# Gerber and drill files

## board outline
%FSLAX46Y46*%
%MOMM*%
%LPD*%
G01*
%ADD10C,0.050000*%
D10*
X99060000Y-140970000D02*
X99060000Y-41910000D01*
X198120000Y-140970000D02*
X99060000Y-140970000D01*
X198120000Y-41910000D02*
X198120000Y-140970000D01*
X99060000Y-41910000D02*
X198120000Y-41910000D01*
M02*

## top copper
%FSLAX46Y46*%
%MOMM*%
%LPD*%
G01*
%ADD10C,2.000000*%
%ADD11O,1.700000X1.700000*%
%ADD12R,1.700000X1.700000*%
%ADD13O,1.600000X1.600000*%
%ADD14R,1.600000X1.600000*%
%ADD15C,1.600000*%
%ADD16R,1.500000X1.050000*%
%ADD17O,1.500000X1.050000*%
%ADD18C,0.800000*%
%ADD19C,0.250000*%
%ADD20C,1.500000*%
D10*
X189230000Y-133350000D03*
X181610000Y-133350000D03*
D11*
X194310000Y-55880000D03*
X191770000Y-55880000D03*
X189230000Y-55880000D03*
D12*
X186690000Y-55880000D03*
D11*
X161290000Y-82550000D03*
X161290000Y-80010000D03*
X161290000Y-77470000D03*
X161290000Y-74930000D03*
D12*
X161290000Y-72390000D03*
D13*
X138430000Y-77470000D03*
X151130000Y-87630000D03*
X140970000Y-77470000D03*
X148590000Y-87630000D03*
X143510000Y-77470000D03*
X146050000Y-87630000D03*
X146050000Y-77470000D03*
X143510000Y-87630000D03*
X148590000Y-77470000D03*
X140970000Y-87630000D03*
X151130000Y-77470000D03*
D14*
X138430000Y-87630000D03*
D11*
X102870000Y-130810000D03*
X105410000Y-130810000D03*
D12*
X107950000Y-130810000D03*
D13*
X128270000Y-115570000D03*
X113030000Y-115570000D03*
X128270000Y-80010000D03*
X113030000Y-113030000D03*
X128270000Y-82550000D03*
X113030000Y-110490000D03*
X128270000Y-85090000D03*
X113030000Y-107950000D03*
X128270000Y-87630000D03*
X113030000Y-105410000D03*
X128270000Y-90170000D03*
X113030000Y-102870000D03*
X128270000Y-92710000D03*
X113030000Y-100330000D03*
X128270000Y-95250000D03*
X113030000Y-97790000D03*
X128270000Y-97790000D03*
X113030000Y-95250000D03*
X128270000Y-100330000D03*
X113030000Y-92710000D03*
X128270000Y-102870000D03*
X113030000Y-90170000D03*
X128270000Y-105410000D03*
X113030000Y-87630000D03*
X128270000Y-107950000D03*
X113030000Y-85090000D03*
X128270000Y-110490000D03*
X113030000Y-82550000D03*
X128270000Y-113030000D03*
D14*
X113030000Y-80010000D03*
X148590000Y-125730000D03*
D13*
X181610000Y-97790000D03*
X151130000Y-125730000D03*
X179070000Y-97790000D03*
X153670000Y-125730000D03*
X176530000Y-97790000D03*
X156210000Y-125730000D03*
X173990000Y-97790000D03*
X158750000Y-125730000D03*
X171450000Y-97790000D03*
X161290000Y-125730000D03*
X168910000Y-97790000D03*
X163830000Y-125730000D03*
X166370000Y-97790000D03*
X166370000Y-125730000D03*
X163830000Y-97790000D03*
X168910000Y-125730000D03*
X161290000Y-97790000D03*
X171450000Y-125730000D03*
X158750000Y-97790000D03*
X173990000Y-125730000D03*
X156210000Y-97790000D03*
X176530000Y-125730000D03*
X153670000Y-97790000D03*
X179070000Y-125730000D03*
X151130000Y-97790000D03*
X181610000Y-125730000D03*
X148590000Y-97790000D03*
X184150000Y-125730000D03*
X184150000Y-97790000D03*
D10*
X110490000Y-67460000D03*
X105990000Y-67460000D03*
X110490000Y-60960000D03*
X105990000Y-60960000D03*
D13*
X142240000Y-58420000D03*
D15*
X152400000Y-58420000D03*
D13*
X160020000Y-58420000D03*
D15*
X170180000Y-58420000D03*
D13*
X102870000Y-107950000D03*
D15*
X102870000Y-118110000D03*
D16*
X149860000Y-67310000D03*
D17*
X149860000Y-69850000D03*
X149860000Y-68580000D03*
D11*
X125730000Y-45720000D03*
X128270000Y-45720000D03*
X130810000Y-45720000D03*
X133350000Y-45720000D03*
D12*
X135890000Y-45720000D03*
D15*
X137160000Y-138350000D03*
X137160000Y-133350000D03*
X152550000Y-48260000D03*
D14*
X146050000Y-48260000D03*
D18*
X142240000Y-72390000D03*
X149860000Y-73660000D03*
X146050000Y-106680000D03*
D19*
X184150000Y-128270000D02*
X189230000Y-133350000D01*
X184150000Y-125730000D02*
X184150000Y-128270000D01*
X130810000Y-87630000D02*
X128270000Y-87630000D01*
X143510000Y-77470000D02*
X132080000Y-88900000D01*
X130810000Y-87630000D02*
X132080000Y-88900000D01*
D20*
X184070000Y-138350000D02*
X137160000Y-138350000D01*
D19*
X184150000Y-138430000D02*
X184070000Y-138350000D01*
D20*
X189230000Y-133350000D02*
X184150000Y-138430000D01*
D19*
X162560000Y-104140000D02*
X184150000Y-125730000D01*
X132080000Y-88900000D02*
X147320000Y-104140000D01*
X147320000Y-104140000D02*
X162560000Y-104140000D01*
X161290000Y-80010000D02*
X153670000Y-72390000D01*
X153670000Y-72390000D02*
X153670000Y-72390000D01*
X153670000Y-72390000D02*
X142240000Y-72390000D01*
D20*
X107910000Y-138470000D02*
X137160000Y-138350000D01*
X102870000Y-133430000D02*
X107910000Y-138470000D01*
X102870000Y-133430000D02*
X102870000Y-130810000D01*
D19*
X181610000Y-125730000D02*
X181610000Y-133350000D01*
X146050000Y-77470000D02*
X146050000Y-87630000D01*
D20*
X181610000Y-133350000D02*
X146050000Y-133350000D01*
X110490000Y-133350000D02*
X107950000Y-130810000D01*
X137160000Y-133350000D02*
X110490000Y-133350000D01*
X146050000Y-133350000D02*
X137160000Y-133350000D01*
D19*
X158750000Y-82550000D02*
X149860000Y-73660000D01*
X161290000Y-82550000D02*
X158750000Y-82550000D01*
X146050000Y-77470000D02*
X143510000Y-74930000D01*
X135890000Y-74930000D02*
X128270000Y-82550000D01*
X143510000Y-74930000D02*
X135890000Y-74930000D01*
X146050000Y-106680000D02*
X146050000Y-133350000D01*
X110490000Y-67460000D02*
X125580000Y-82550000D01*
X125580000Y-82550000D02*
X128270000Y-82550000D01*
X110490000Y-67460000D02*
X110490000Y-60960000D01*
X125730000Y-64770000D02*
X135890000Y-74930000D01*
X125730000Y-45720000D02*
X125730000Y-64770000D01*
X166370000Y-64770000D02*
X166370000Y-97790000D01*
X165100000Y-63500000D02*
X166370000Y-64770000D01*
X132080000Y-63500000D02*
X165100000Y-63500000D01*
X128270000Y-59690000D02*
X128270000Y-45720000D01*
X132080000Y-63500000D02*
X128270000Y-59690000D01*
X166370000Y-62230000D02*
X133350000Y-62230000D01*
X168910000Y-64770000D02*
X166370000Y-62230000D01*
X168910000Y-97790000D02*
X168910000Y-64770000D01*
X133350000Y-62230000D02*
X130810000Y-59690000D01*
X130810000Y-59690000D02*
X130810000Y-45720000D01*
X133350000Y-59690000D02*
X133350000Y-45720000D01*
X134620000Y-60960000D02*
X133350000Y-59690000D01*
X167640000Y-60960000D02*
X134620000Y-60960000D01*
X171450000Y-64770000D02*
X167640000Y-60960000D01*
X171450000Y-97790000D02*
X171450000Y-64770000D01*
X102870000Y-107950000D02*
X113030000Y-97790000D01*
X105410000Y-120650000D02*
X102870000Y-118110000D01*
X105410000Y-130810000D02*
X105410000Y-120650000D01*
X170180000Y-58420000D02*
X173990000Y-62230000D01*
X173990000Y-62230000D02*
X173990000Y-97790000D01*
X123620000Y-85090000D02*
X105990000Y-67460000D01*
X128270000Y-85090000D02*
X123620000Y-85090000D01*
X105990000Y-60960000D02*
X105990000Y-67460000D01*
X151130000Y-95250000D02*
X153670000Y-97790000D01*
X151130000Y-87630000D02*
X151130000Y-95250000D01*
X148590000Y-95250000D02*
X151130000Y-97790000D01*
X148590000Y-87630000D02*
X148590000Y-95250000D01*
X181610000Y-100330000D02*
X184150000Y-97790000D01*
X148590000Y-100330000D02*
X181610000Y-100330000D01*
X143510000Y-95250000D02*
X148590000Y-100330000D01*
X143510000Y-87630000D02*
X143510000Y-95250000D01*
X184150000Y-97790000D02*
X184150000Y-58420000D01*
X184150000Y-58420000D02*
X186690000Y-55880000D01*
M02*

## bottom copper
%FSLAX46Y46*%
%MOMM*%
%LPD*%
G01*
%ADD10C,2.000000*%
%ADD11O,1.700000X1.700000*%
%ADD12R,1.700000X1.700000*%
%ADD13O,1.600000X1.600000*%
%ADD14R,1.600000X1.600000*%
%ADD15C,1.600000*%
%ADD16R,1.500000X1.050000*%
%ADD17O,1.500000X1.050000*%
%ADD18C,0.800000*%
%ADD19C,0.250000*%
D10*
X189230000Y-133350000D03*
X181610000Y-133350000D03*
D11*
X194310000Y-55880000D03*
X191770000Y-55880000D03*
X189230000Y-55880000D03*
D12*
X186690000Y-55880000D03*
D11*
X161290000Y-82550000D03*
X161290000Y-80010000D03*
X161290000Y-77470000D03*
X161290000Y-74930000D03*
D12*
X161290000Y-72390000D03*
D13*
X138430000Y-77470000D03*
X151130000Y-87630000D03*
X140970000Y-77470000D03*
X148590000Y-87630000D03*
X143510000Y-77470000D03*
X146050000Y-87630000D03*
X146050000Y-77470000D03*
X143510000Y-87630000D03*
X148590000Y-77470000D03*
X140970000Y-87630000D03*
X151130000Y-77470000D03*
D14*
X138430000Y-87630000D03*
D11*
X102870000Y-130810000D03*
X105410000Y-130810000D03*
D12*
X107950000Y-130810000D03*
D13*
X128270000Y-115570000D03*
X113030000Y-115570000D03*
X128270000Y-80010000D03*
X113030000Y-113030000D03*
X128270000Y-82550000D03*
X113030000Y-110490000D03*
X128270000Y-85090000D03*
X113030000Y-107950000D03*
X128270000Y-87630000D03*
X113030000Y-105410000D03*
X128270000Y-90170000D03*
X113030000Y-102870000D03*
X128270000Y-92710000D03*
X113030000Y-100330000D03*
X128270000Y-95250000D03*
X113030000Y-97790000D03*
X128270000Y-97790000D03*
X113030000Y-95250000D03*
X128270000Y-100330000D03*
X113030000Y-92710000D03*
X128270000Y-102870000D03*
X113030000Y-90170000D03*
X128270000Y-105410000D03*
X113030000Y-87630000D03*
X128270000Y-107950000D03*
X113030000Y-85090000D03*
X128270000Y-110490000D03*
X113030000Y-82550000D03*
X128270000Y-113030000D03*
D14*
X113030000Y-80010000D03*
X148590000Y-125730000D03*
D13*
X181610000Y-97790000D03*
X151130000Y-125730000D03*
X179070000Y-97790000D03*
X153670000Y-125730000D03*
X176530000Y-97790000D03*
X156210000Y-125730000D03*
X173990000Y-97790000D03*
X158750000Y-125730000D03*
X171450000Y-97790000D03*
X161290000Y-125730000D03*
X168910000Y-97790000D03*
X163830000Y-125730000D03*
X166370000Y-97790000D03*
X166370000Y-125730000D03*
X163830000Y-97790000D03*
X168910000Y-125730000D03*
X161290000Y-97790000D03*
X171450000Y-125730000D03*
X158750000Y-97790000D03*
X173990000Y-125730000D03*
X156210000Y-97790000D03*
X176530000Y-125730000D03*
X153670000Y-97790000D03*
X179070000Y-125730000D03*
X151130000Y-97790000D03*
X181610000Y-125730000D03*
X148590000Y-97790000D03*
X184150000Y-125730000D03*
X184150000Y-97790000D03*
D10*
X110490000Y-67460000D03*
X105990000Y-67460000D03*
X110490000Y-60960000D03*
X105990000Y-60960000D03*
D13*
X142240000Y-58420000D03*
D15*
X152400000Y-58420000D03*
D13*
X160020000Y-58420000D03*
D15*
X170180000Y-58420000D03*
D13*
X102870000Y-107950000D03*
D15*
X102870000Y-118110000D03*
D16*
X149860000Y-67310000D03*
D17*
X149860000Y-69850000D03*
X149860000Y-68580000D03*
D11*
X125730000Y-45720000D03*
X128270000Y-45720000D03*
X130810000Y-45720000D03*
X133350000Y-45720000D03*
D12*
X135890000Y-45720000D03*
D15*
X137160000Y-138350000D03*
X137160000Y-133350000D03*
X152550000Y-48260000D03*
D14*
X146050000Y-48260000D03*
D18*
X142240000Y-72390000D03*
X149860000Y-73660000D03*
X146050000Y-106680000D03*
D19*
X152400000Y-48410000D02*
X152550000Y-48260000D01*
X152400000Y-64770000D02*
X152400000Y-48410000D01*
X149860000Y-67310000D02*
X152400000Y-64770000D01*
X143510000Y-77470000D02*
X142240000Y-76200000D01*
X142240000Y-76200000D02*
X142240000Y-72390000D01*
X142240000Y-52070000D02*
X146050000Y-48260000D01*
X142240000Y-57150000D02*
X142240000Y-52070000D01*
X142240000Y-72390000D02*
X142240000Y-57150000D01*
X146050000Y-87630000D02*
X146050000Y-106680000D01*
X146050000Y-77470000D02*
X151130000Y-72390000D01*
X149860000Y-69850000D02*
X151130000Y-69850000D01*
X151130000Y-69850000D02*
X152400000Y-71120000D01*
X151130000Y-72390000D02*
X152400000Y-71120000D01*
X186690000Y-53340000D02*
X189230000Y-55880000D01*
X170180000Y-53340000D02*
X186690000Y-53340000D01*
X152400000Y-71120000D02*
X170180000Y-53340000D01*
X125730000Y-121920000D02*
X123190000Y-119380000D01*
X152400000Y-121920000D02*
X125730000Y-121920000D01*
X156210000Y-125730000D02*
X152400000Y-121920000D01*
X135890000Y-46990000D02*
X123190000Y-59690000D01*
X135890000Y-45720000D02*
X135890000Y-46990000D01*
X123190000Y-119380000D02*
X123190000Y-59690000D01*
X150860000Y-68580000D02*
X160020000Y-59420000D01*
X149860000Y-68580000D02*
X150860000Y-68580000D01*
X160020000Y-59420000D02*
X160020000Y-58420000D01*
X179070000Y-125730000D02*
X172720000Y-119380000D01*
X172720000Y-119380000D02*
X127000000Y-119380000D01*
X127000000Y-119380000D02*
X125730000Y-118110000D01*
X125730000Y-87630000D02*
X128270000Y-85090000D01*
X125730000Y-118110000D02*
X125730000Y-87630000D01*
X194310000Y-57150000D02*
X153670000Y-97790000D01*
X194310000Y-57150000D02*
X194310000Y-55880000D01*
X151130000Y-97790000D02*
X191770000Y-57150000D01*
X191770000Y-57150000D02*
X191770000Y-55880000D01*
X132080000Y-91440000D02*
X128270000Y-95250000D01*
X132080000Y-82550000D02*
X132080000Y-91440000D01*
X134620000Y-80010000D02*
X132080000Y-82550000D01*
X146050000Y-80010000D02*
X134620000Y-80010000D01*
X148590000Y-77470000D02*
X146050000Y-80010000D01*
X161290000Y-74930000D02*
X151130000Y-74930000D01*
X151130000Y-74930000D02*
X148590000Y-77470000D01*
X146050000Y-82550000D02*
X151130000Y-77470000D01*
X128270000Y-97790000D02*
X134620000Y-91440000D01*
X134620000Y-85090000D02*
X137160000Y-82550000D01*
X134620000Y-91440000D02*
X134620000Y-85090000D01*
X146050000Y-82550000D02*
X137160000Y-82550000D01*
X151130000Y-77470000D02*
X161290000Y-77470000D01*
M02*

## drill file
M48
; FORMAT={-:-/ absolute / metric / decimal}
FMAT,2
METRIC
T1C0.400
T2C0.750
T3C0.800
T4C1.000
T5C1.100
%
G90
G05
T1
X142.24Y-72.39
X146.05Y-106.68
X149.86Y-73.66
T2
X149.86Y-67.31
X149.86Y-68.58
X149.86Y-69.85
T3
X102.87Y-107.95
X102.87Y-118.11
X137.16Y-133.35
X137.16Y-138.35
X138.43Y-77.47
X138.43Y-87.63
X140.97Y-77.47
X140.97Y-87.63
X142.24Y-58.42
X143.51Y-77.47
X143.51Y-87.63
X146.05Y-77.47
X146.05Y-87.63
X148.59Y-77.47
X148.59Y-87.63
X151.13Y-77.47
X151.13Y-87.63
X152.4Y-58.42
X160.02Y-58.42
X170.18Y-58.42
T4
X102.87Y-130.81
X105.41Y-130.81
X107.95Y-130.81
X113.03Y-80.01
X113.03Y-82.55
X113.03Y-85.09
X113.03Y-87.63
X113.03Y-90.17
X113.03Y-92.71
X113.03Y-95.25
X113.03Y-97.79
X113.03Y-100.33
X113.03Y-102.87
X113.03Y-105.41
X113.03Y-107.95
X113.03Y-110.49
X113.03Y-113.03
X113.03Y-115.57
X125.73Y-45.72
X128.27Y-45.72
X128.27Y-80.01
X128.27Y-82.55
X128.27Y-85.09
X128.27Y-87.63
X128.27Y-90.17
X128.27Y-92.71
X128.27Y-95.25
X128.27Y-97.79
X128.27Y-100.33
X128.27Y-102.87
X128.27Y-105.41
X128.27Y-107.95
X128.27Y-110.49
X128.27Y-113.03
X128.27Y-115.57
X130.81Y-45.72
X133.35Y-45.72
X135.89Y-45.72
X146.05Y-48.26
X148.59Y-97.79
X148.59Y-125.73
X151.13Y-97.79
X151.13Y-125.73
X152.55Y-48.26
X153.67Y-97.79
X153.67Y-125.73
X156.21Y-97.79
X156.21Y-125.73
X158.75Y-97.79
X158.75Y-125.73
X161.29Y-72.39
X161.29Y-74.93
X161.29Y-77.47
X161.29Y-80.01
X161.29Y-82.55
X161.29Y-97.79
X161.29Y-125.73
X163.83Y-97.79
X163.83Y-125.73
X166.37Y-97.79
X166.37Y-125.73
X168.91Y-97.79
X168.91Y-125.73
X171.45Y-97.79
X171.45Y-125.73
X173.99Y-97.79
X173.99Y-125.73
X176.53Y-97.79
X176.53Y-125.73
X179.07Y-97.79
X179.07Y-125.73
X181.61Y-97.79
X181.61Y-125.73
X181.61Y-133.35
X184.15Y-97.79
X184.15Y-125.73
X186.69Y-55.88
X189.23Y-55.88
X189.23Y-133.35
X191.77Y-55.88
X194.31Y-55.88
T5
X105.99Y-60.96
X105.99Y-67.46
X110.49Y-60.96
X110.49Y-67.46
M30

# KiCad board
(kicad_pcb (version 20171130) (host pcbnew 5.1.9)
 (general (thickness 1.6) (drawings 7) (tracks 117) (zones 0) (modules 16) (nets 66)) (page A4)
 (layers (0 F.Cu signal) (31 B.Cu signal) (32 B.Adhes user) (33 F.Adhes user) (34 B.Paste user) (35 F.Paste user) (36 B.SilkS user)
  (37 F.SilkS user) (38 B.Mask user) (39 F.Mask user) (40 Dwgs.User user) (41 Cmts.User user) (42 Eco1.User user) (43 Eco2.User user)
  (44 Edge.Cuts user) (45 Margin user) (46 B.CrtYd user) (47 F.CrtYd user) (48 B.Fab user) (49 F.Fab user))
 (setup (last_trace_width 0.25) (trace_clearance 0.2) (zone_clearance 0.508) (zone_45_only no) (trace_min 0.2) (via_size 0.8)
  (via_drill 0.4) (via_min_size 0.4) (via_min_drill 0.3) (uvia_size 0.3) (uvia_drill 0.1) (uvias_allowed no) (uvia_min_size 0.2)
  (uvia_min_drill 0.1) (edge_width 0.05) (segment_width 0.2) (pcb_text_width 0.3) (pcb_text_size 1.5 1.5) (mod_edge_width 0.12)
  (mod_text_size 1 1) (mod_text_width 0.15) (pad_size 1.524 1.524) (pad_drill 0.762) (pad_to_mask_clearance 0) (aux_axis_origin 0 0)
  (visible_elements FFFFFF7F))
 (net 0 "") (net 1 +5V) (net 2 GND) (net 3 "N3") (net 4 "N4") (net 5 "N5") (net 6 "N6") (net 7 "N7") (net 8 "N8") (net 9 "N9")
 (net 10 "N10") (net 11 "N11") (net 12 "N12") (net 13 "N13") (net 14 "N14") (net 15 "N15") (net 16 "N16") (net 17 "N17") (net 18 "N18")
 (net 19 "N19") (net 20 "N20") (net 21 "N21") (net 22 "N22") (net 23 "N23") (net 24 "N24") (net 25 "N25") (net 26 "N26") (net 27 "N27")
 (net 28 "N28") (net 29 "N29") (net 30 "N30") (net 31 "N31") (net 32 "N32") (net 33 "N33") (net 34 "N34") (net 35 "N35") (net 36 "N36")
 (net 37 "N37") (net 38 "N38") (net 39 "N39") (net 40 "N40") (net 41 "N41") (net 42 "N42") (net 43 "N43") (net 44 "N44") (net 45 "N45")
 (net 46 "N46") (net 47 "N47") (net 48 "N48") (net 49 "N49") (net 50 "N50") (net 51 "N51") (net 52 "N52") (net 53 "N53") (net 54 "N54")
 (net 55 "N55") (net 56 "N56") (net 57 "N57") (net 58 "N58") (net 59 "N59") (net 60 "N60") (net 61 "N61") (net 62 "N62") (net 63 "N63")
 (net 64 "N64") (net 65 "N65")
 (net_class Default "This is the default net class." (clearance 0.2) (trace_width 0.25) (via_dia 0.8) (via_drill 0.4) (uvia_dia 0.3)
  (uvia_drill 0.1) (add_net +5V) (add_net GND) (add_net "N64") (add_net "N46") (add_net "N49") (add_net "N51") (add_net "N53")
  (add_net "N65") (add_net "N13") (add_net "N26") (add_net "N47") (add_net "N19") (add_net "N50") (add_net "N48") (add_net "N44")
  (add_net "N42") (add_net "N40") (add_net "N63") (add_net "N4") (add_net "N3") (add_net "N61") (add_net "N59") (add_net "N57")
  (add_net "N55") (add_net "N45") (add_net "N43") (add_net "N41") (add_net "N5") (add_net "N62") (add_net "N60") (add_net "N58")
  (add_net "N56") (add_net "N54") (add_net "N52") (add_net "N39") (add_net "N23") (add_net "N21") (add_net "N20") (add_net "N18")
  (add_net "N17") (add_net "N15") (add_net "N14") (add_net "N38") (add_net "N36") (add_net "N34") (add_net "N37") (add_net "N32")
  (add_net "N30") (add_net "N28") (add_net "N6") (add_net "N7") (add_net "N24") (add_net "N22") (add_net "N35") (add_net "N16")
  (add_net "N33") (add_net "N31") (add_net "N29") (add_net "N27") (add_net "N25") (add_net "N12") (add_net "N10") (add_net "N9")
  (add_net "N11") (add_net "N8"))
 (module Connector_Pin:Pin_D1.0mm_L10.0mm (layer F.Cu) (at 189.23 133.35)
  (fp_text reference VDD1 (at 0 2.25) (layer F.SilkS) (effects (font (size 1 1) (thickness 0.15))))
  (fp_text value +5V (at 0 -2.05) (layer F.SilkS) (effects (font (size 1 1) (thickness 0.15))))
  (pad 1 thru_hole circle (at 0 0) (size 2 2) (drill 1) (layers *.Cu *.Mask) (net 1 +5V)))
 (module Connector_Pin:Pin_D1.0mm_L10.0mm (layer F.Cu) (at 181.61 133.35)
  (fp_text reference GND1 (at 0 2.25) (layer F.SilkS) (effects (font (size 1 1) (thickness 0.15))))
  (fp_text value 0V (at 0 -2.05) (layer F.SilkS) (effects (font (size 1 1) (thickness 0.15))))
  (pad 1 thru_hole circle (at 0 0) (size 2 2) (drill 1) (layers *.Cu *.Mask) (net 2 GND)))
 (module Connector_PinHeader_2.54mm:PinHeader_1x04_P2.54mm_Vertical (layer F.Cu) (at 186.69 55.88 90)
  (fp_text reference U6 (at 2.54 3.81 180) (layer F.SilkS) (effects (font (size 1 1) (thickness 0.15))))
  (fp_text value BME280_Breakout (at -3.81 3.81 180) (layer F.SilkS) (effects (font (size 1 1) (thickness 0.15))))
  (pad 4 thru_hole oval (at 0 7.62 90) (size 1.7 1.7) (drill 1) (layers *.Cu *.Mask) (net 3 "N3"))
  (pad 3 thru_hole oval (at 0 5.08 90) (size 1.7 1.7) (drill 1) (layers *.Cu *.Mask) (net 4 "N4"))
  (pad 2 thru_hole oval (at 0 2.54 90) (size 1.7 1.7) (drill 1) (layers *.Cu *.Mask) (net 2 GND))
  (pad 1 thru_hole rect (at 0 0 90) (size 1.7 1.7) (drill 1) (layers *.Cu *.Mask) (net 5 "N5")))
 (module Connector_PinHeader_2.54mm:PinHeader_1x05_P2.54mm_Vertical (layer F.Cu) (at 161.29 72.39)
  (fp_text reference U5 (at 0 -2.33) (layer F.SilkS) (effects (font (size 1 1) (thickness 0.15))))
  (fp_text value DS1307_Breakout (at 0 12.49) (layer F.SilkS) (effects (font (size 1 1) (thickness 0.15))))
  (pad 5 thru_hole oval (at 0 10.16) (size 1.7 1.7) (drill 1) (layers *.Cu *.Mask) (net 2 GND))
  (pad 4 thru_hole oval (at 0 7.62) (size 1.7 1.7) (drill 1) (layers *.Cu *.Mask) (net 1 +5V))
  (pad 3 thru_hole oval (at 0 5.08) (size 1.7 1.7) (drill 1) (layers *.Cu *.Mask) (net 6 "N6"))
  (pad 2 thru_hole oval (at 0 2.54) (size 1.7 1.7) (drill 1) (layers *.Cu *.Mask) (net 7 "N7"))
  (pad 1 thru_hole rect (at 0 0) (size 1.7 1.7) (drill 1) (layers *.Cu *.Mask) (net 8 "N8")))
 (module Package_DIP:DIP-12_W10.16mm (layer F.Cu) (at 138.43 87.63 90)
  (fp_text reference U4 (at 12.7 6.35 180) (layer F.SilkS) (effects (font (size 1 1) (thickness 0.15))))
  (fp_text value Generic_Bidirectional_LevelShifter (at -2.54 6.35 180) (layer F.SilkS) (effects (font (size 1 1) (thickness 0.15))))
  (pad 12 thru_hole oval (at 10.16 0 90) (size 1.6 1.6) (drill 0.8) (layers *.Cu *.Mask) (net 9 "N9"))
  (pad 6 thru_hole oval (at 0 12.7 90) (size 1.6 1.6) (drill 0.8) (layers *.Cu *.Mask) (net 3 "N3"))
  (pad 11 thru_hole oval (at 10.16 2.54 90) (size 1.6 1.6) (drill 0.8) (layers *.Cu *.Mask) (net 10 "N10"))
  (pad 5 thru_hole oval (at 0 10.16 90) (size 1.6 1.6) (drill 0.8) (layers *.Cu *.Mask) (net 4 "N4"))
  (pad 10 thru_hole oval (at 10.16 5.08 90) (size 1.6 1.6) (drill 0.8) (layers *.Cu *.Mask) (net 1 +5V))
  (pad 4 thru_hole oval (at 0 7.62 90) (size 1.6 1.6) (drill 0.8) (layers *.Cu *.Mask) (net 2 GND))
  (pad 9 thru_hole oval (at 10.16 7.62 90) (size 1.6 1.6) (drill 0.8) (layers *.Cu *.Mask) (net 2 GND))
  (pad 3 thru_hole oval (at 0 5.08 90) (size 1.6 1.6) (drill 0.8) (layers *.Cu *.Mask) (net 5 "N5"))
  (pad 8 thru_hole oval (at 10.16 10.16 90) (size 1.6 1.6) (drill 0.8) (layers *.Cu *.Mask) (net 7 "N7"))
  (pad 2 thru_hole oval (at 0 2.54 90) (size 1.6 1.6) (drill 0.8) (layers *.Cu *.Mask) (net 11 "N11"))
  (pad 7 thru_hole oval (at 10.16 12.7 90) (size 1.6 1.6) (drill 0.8) (layers *.Cu *.Mask) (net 6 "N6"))
  (pad 1 thru_hole rect (at 0 0 90) (size 1.6 1.6) (drill 0.8) (layers *.Cu *.Mask) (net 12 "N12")))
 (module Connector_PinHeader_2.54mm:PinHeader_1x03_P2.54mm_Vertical (layer F.Cu) (at 107.95 130.81 270)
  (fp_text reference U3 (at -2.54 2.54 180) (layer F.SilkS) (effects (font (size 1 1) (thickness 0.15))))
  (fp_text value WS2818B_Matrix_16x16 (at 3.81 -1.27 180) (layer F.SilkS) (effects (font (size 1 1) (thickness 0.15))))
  (pad 3 thru_hole oval (at 0 5.08 270) (size 1.7 1.7) (drill 1) (layers *.Cu *.Mask) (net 1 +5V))
  (pad 2 thru_hole oval (at 0 2.54 270) (size 1.7 1.7) (drill 1) (layers *.Cu *.Mask) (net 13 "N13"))
  (pad 1 thru_hole rect (at 0 0 270) (size 1.7 1.7) (drill 1) (layers *.Cu *.Mask) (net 2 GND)))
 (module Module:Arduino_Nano (layer F.Cu) (at 113.03 80.01)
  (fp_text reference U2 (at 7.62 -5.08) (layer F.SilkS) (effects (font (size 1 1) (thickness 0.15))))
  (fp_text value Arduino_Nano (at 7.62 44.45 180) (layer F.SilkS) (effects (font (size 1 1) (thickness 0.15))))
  (pad 16 thru_hole oval (at 15.24 35.56) (size 1.6 1.6) (drill 1) (layers *.Cu *.Mask) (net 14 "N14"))
  (pad 15 thru_hole oval (at 0 35.56) (size 1.6 1.6) (drill 1) (layers *.Cu *.Mask) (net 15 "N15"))
  (pad 30 thru_hole oval (at 15.24 0) (size 1.6 1.6) (drill 1) (layers *.Cu *.Mask) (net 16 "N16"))
  (pad 14 thru_hole oval (at 0 33.02) (size 1.6 1.6) (drill 1) (layers *.Cu *.Mask) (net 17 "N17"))
  (pad 29 thru_hole oval (at 15.24 2.54) (size 1.6 1.6) (drill 1) (layers *.Cu *.Mask) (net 2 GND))
  (pad 13 thru_hole oval (at 0 30.48) (size 1.6 1.6) (drill 1) (layers *.Cu *.Mask) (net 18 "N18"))
  (pad 28 thru_hole oval (at 15.24 5.08) (size 1.6 1.6) (drill 1) (layers *.Cu *.Mask) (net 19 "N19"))
  (pad 12 thru_hole oval (at 0 27.94) (size 1.6 1.6) (drill 1) (layers *.Cu *.Mask) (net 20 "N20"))
  (pad 27 thru_hole oval (at 15.24 7.62) (size 1.6 1.6) (drill 1) (layers *.Cu *.Mask) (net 1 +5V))
  (pad 11 thru_hole oval (at 0 25.4) (size 1.6 1.6) (drill 1) (layers *.Cu *.Mask) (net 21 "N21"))
  (pad 26 thru_hole oval (at 15.24 10.16) (size 1.6 1.6) (drill 1) (layers *.Cu *.Mask) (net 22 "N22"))
  (pad 10 thru_hole oval (at 0 22.86) (size 1.6 1.6) (drill 1) (layers *.Cu *.Mask) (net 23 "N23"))
  (pad 25 thru_hole oval (at 15.24 12.7) (size 1.6 1.6) (drill 1) (layers *.Cu *.Mask) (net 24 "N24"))
  (pad 9 thru_hole oval (at 0 20.32) (size 1.6 1.6) (drill 1) (layers *.Cu *.Mask) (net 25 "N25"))
  (pad 24 thru_hole oval (at 15.24 15.24) (size 1.6 1.6) (drill 1) (layers *.Cu *.Mask) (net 7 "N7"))
  (pad 8 thru_hole oval (at 0 17.78) (size 1.6 1.6) (drill 1) (layers *.Cu *.Mask) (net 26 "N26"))
  (pad 23 thru_hole oval (at 15.24 17.78) (size 1.6 1.6) (drill 1) (layers *.Cu *.Mask) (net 6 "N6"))
  (pad 7 thru_hole oval (at 0 15.24) (size 1.6 1.6) (drill 1) (layers *.Cu *.Mask) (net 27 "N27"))
  (pad 22 thru_hole oval (at 15.24 20.32) (size 1.6 1.6) (drill 1) (layers *.Cu *.Mask) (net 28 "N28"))
  (pad 6 thru_hole oval (at 0 12.7) (size 1.6 1.6) (drill 1) (layers *.Cu *.Mask) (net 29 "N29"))
  (pad 21 thru_hole oval (at 15.24 22.86) (size 1.6 1.6) (drill 1) (layers *.Cu *.Mask) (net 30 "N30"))
  (pad 5 thru_hole oval (at 0 10.16) (size 1.6 1.6) (drill 1) (layers *.Cu *.Mask) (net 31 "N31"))
  (pad 20 thru_hole oval (at 15.24 25.4) (size 1.6 1.6) (drill 1) (layers *.Cu *.Mask) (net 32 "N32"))
  (pad 4 thru_hole oval (at 0 7.62) (size 1.6 1.6) (drill 1) (layers *.Cu *.Mask) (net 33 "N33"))
  (pad 19 thru_hole oval (at 15.24 27.94) (size 1.6 1.6) (drill 1) (layers *.Cu *.Mask) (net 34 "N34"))
  (pad 3 thru_hole oval (at 0 5.08) (size 1.6 1.6) (drill 1) (layers *.Cu *.Mask) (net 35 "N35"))
  (pad 18 thru_hole oval (at 15.24 30.48) (size 1.6 1.6) (drill 1) (layers *.Cu *.Mask) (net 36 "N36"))
  (pad 2 thru_hole oval (at 0 2.54) (size 1.6 1.6) (drill 1) (layers *.Cu *.Mask) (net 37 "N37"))
  (pad 17 thru_hole oval (at 15.24 33.02) (size 1.6 1.6) (drill 1) (layers *.Cu *.Mask) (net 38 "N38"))
  (pad 1 thru_hole rect (at 0 0) (size 1.6 1.6) (drill 1) (layers *.Cu *.Mask) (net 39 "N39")))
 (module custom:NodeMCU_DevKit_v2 (layer F.Cu) (at 148.59 125.73 90)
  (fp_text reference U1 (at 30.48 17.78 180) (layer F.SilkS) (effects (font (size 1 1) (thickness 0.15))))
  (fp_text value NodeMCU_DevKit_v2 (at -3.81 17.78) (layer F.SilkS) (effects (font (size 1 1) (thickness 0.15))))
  (pad 15 thru_hole rect (at 0 0 90) (size 1.6 1.6) (drill 1) (layers *.Cu *.Mask) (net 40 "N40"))
  (pad 29 thru_hole oval (at 27.94 33.02 90) (size 1.6 1.6) (drill 1) (layers *.Cu *.Mask) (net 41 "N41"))
  (pad 14 thru_hole oval (at 0 2.54 90) (size 1.6 1.6) (drill 1) (layers *.Cu *.Mask) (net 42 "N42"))
  (pad 28 thru_hole oval (at 27.94 30.48 90) (size 1.6 1.6) (drill 1) (layers *.Cu *.Mask) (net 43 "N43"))
  (pad 13 thru_hole oval (at 0 5.08 90) (size 1.6 1.6) (drill 1) (layers *.Cu *.Mask) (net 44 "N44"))
  (pad 27 thru_hole oval (at 27.94 27.94 90) (size 1.6 1.6) (drill 1) (layers *.Cu *.Mask) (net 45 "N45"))
  (pad 12 thru_hole oval (at 0 7.62 90) (size 1.6 1.6) (drill 1) (layers *.Cu *.Mask) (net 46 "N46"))
  (pad 26 thru_hole oval (at 27.94 25.4 90) (size 1.6 1.6) (drill 1) (layers *.Cu *.Mask) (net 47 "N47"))
  (pad 11 thru_hole oval (at 0 10.16 90) (size 1.6 1.6) (drill 1) (layers *.Cu *.Mask) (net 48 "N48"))
  (pad 25 thru_hole oval (at 27.94 22.86 90) (size 1.6 1.6) (drill 1) (layers *.Cu *.Mask) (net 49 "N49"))
  (pad 10 thru_hole oval (at 0 12.7 90) (size 1.6 1.6) (drill 1) (layers *.Cu *.Mask) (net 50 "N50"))
  (pad 24 thru_hole oval (at 27.94 20.32 90) (size 1.6 1.6) (drill 1) (layers *.Cu *.Mask) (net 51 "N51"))
  (pad 9 thru_hole oval (at 0 15.24 90) (size 1.6 1.6) (drill 1) (layers *.Cu *.Mask) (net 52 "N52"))
  (pad 23 thru_hole oval (at 27.94 17.78 90) (size 1.6 1.6) (drill 1) (layers *.Cu *.Mask) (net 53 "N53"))
  (pad 8 thru_hole oval (at 0 17.78 90) (size 1.6 1.6) (drill 1) (layers *.Cu *.Mask) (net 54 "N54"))
  (pad 22 thru_hole oval (at 27.94 15.24 90) (size 1.6 1.6) (drill 1) (layers *.Cu *.Mask) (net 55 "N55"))
  (pad 7 thru_hole oval (at 0 20.32 90) (size 1.6 1.6) (drill 1) (layers *.Cu *.Mask) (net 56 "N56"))
  (pad 21 thru_hole oval (at 27.94 12.7 90) (size 1.6 1.6) (drill 1) (layers *.Cu *.Mask) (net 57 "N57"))
  (pad 6 thru_hole oval (at 0 22.86 90) (size 1.6 1.6) (drill 1) (layers *.Cu *.Mask) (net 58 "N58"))
  (pad 20 thru_hole oval (at 27.94 10.16 90) (size 1.6 1.6) (drill 1) (layers *.Cu *.Mask) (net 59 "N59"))
  (pad 5 thru_hole oval (at 0 25.4 90) (size 1.6 1.6) (drill 1) (layers *.Cu *.Mask) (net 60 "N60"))
  (pad 19 thru_hole oval (at 27.94 7.62 90) (size 1.6 1.6) (drill 1) (layers *.Cu *.Mask) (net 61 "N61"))
  (pad 4 thru_hole oval (at 0 27.94 90) (size 1.6 1.6) (drill 1) (layers *.Cu *.Mask) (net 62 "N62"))
  (pad 18 thru_hole oval (at 27.94 5.08 90) (size 1.6 1.6) (drill 1) (layers *.Cu *.Mask) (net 3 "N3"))
  (pad 3 thru_hole oval (at 0 30.48 90) (size 1.6 1.6) (drill 1) (layers *.Cu *.Mask) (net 19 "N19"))
  (pad 17 thru_hole oval (at 27.94 2.54 90) (size 1.6 1.6) (drill 1) (layers *.Cu *.Mask) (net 4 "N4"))
  (pad 2 thru_hole oval (at 0 33.02 90) (size 1.6 1.6) (drill 1) (layers *.Cu *.Mask) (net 2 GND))
  (pad 16 thru_hole oval (at 27.94 0 90) (size 1.6 1.6) (drill 1) (layers *.Cu *.Mask) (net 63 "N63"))
  (pad 1 thru_hole oval (at 0 35.56 90) (size 1.6 1.6) (drill 1) (layers *.Cu *.Mask) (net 1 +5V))
  (pad 30 thru_hole oval (at 27.94 35.56 90) (size 1.6 1.6) (drill 1) (layers *.Cu *.Mask) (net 5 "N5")))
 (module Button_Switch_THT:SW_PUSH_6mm (layer F.Cu) (at 110.49 60.96 270)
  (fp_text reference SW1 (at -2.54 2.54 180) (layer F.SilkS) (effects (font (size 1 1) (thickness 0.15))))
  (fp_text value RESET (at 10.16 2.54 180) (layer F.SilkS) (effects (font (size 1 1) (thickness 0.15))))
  (pad 1 thru_hole circle (at 6.5 0) (size 2 2) (drill 1.1) (layers *.Cu *.Mask) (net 2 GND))
  (pad 2 thru_hole circle (at 6.5 4.5) (size 2 2) (drill 1.1) (layers *.Cu *.Mask) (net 19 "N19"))
  (pad 1 thru_hole circle (at 0 0) (size 2 2) (drill 1.1) (layers *.Cu *.Mask) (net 2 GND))
  (pad 2 thru_hole circle (at 0 4.5) (size 2 2) (drill 1.1) (layers *.Cu *.Mask) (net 19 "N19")))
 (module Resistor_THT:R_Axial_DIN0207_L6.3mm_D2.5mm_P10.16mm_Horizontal (layer F.Cu) (at 152.4 58.42 180)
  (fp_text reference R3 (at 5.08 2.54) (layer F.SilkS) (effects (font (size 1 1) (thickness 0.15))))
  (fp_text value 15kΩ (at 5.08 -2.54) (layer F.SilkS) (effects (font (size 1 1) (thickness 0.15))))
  (pad 2 thru_hole oval (at 10.16 0 180) (size 1.6 1.6) (drill 0.8) (layers *.Cu *.Mask) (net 1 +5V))
  (pad 1 thru_hole circle (at 0 0 180) (size 1.6 1.6) (drill 0.8) (layers *.Cu *.Mask) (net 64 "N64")))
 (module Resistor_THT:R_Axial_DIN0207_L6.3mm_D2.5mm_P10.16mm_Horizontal (layer F.Cu) (at 170.18 58.42 180)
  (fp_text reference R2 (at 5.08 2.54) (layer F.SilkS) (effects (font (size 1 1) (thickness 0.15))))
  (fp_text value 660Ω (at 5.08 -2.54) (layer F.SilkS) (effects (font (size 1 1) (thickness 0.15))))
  (pad 2 thru_hole oval (at 10.16 0 180) (size 1.6 1.6) (drill 0.8) (layers *.Cu *.Mask) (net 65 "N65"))
  (pad 1 thru_hole circle (at 0 0 180) (size 1.6 1.6) (drill 0.8) (layers *.Cu *.Mask) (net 47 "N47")))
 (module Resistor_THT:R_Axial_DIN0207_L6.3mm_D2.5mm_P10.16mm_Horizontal (layer F.Cu) (at 102.87 118.11 90)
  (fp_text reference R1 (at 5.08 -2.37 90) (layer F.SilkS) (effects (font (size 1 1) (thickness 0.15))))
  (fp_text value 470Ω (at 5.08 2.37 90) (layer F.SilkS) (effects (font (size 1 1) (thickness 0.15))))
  (pad 2 thru_hole oval (at 10.16 0 90) (size 1.6 1.6) (drill 0.8) (layers *.Cu *.Mask) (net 26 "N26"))
  (pad 1 thru_hole circle (at 0 0 90) (size 1.6 1.6) (drill 0.8) (layers *.Cu *.Mask) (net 13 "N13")))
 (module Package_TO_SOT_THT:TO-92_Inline (layer F.Cu) (at 149.86 67.31 270)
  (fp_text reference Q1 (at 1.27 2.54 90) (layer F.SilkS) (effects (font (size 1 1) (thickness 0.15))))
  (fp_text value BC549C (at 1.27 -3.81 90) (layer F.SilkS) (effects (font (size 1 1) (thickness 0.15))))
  (pad 1 thru_hole rect (at 0 0 270) (size 1.05 1.5) (drill 0.75) (layers *.Cu *.Mask) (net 64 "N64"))
  (pad 3 thru_hole oval (at 2.54 0 270) (size 1.05 1.5) (drill 0.75) (layers *.Cu *.Mask) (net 2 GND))
  (pad 2 thru_hole oval (at 1.27 0 270) (size 1.05 1.5) (drill 0.75) (layers *.Cu *.Mask) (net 65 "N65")))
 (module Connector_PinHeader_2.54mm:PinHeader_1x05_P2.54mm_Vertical (layer F.Cu) (at 135.89 45.72 270)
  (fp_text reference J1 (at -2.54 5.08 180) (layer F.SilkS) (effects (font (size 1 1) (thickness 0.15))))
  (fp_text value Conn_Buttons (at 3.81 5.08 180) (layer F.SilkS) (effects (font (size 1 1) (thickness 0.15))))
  (pad 5 thru_hole oval (at 0 10.16 270) (size 1.7 1.7) (drill 1) (layers *.Cu *.Mask) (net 2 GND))
  (pad 4 thru_hole oval (at 0 7.62 270) (size 1.7 1.7) (drill 1) (layers *.Cu *.Mask) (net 53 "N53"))
  (pad 3 thru_hole oval (at 0 5.08 270) (size 1.7 1.7) (drill 1) (layers *.Cu *.Mask) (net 51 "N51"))
  (pad 2 thru_hole oval (at 0 2.54 270) (size 1.7 1.7) (drill 1) (layers *.Cu *.Mask) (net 49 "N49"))
  (pad 1 thru_hole rect (at 0 0 270) (size 1.7 1.7) (drill 1) (layers *.Cu *.Mask) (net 46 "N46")))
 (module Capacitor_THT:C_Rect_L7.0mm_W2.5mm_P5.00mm (layer F.Cu) (at 137.16 133.35 270)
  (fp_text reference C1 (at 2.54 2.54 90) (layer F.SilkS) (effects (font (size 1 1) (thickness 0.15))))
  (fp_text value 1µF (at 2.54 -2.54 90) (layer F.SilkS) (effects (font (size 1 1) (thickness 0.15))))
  (pad 2 thru_hole circle (at 5 0 270) (size 1.6 1.6) (drill 0.8) (layers *.Cu *.Mask) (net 1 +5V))
  (pad 1 thru_hole circle (at 0 0 270) (size 1.6 1.6) (drill 0.8) (layers *.Cu *.Mask) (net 2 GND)))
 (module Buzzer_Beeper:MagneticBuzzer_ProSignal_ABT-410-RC (layer F.Cu) (at 146.05 48.26)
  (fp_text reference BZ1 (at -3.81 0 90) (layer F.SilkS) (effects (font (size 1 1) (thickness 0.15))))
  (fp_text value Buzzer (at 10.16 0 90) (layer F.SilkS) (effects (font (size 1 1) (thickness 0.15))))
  (pad 2 thru_hole circle (at 6.5 0) (size 1.6 1.6) (drill 1) (layers *.Cu *.Mask) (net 64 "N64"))
  (pad 1 thru_hole rect (at 0 0) (size 1.6 1.6) (drill 1) (layers *.Cu *.Mask) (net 1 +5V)))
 (gr_line (start 99.06 140.97) (end 99.06 41.91) (layer Edge.Cuts) (width 0.05))
 (gr_line (start 198.12 140.97) (end 99.06 140.97) (layer Edge.Cuts) (width 0.05))
 (gr_line (start 198.12 41.91) (end 198.12 140.97) (layer Edge.Cuts) (width 0.05))
 (gr_line (start 99.06 41.91) (end 198.12 41.91) (layer Edge.Cuts) (width 0.05))
 (segment (start 152.4 48.41) (end 152.55 48.26) (width 0.25) (layer B.Cu) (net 64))
 (segment (start 152.4 64.77) (end 152.4 48.41) (width 0.25) (layer B.Cu) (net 64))
 (segment (start 149.86 67.31) (end 152.4 64.77) (width 0.25) (layer B.Cu) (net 64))
 (segment (start 184.15 128.27) (end 189.23 133.35) (width 0.25) (layer F.Cu) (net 1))
 (segment (start 184.15 125.73) (end 184.15 128.27) (width 0.25) (layer F.Cu) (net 1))
 (segment (start 130.81 87.63) (end 128.27 87.63) (width 0.25) (layer F.Cu) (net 1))
 (segment (start 143.51 77.47) (end 132.08 88.9) (width 0.25) (layer F.Cu) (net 1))
 (segment (start 130.81 87.63) (end 132.08 88.9) (width 0.25) (layer F.Cu) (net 1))
 (segment (start 184.07 138.35) (end 137.16 138.35) (width 1.5) (layer F.Cu) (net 1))
 (segment (start 184.15 138.43) (end 184.07 138.35) (width 0.25) (layer F.Cu) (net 1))
 (segment (start 189.23 133.35) (end 184.15 138.43) (width 1.5) (layer F.Cu) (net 1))
 (segment (start 162.56 104.14) (end 184.15 125.73) (width 0.25) (layer F.Cu) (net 1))
 (segment (start 132.08 88.9) (end 147.32 104.14) (width 0.25) (layer F.Cu) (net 1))
 (segment (start 147.32 104.14) (end 162.56 104.14) (width 0.25) (layer F.Cu) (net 1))
 (segment (start 143.51 77.47) (end 142.24 76.2) (width 0.25) (layer B.Cu) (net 1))
 (segment (start 142.24 76.2) (end 142.24 72.39) (width 0.25) (layer B.Cu) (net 1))
 (segment (start 142.24 52.07) (end 146.05 48.26) (width 0.25) (layer B.Cu) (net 1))
 (segment (start 161.29 80.01) (end 153.67 72.39) (width 0.25) (layer F.Cu) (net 1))
 (segment (start 153.67 72.39) (end 153.67 72.39) (width 0.25) (layer F.Cu) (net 1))
 (via (at 142.24 72.39) (size 0.8) (drill 0.4) (layers F.Cu B.Cu) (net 1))
 (segment (start 153.67 72.39) (end 142.24 72.39) (width 0.25) (layer F.Cu) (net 1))
 (segment (start 107.91 138.47) (end 137.16 138.35) (width 1.5) (layer F.Cu) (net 1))
 (segment (start 102.87 133.43) (end 107.91 138.47) (width 1.5) (layer F.Cu) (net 1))
 (segment (start 102.87 133.43) (end 102.87 130.81) (width 1.5) (layer F.Cu) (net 1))
 (segment (start 142.24 57.15) (end 142.24 52.07) (width 0.25) (layer B.Cu) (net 1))
 (segment (start 142.24 72.39) (end 142.24 57.15) (width 0.25) (layer B.Cu) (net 1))
 (segment (start 181.61 125.73) (end 181.61 133.35) (width 0.25) (layer F.Cu) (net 2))
 (segment (start 146.05 77.47) (end 146.05 87.63) (width 0.25) (layer F.Cu) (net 2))
 (segment (start 181.61 133.35) (end 146.05 133.35) (width 1.5) (layer F.Cu) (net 2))
 (segment (start 110.49 133.35) (end 107.95 130.81) (width 1.5) (layer F.Cu) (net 2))
 (segment (start 137.16 133.35) (end 110.49 133.35) (width 1.5) (layer F.Cu) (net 2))
 (segment (start 146.05 133.35) (end 137.16 133.35) (width 1.5) (layer F.Cu) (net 2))
 (segment (start 146.05 87.63) (end 146.05 106.68) (width 0.25) (layer B.Cu) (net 2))
 (segment (start 146.05 77.47) (end 151.13 72.39) (width 0.25) (layer B.Cu) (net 2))
 (segment (start 149.86 69.85) (end 151.13 69.85) (width 0.25) (layer B.Cu) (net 2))
 (segment (start 151.13 69.85) (end 152.4 71.12) (width 0.25) (layer B.Cu) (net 2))
 (segment (start 151.13 72.39) (end 152.4 71.12) (width 0.25) (layer B.Cu) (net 2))
 (via (at 149.86 73.66) (size 0.8) (drill 0.4) (layers F.Cu B.Cu) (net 2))
 (segment (start 158.75 82.55) (end 149.86 73.66) (width 0.25) (layer F.Cu) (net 2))
 (segment (start 161.29 82.55) (end 158.75 82.55) (width 0.25) (layer F.Cu) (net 2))
 (segment (start 146.05 77.47) (end 143.51 74.93) (width 0.25) (layer F.Cu) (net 2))
 (segment (start 135.89 74.93) (end 128.27 82.55) (width 0.25) (layer F.Cu) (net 2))
 (segment (start 143.51 74.93) (end 135.89 74.93) (width 0.25) (layer F.Cu) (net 2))
 (via (at 146.05 106.68) (size 0.8) (drill 0.4) (layers F.Cu B.Cu) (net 2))
 (segment (start 146.05 106.68) (end 146.05 133.35) (width 0.25) (layer F.Cu) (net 2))
 (segment (start 110.49 67.46) (end 125.58 82.55) (width 0.25) (layer F.Cu) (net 2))
 (segment (start 125.58 82.55) (end 128.27 82.55) (width 0.25) (layer F.Cu) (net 2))
 (segment (start 110.49 67.46) (end 110.49 60.96) (width 0.25) (layer F.Cu) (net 2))
 (segment (start 186.69 53.34) (end 189.23 55.88) (width 0.25) (layer B.Cu) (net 2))
 (segment (start 170.18 53.34) (end 186.69 53.34) (width 0.25) (layer B.Cu) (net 2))
 (segment (start 152.4 71.12) (end 170.18 53.34) (width 0.25) (layer B.Cu) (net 2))
 (segment (start 125.73 64.77) (end 135.89 74.93) (width 0.25) (layer F.Cu) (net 2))
 (segment (start 125.73 45.72) (end 125.73 64.77) (width 0.25) (layer F.Cu) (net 2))
 (segment (start 166.37 64.77) (end 166.37 97.79) (width 0.25) (layer F.Cu) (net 53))
 (segment (start 165.1 63.5) (end 166.37 64.77) (width 0.25) (layer F.Cu) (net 53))
 (segment (start 132.08 63.5) (end 165.1 63.5) (width 0.25) (layer F.Cu) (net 53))
 (segment (start 128.27 59.69) (end 128.27 45.72) (width 0.25) (layer F.Cu) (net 53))
 (segment (start 132.08 63.5) (end 128.27 59.69) (width 0.25) (layer F.Cu) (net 53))
 (segment (start 166.37 62.23) (end 133.35 62.23) (width 0.25) (layer F.Cu) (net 51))
 (segment (start 168.91 64.77) (end 166.37 62.23) (width 0.25) (layer F.Cu) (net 51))
 (segment (start 168.91 97.79) (end 168.91 64.77) (width 0.25) (layer F.Cu) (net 51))
 (segment (start 133.35 62.23) (end 130.81 59.69) (width 0.25) (layer F.Cu) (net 51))
 (segment (start 130.81 59.69) (end 130.81 45.72) (width 0.25) (layer F.Cu) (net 51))
 (segment (start 133.35 59.69) (end 133.35 45.72) (width 0.25) (layer F.Cu) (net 49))
 (segment (start 134.62 60.96) (end 133.35 59.69) (width 0.25) (layer F.Cu) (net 49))
 (segment (start 167.64 60.96) (end 134.62 60.96) (width 0.25) (layer F.Cu) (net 49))
 (segment (start 171.45 64.77) (end 167.64 60.96) (width 0.25) (layer F.Cu) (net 49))
 (segment (start 171.45 97.79) (end 171.45 64.77) (width 0.25) (layer F.Cu) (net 49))
 (segment (start 125.73 121.92) (end 123.19 119.38) (width 0.25) (layer B.Cu) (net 46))
 (segment (start 152.4 121.92) (end 125.73 121.92) (width 0.25) (layer B.Cu) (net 46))
 (segment (start 156.21 125.73) (end 152.4 121.92) (width 0.25) (layer B.Cu) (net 46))
 (segment (start 135.89 46.99) (end 123.19 59.69) (width 0.25) (layer B.Cu) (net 46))
 (segment (start 135.89 45.72) (end 135.89 46.99) (width 0.25) (layer B.Cu) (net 46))
 (segment (start 123.19 119.38) (end 123.19 59.69) (width 0.25) (layer B.Cu) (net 46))
 (segment (start 150.86 68.58) (end 160.02 59.42) (width 0.25) (layer B.Cu) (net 65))
 (segment (start 149.86 68.58) (end 150.86 68.58) (width 0.25) (layer B.Cu) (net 65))
 (segment (start 160.02 59.42) (end 160.02 58.42) (width 0.25) (layer B.Cu) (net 65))
 (segment (start 102.87 107.95) (end 113.03 97.79) (width 0.25) (layer F.Cu) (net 26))
 (segment (start 105.41 120.65) (end 102.87 118.11) (width 0.25) (layer F.Cu) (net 13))
 (segment (start 105.41 130.81) (end 105.41 120.65) (width 0.25) (layer F.Cu) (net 13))
 (segment (start 170.18 58.42) (end 173.99 62.23) (width 0.25) (layer F.Cu) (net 47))
 (segment (start 173.99 62.23) (end 173.99 97.79) (width 0.25) (layer F.Cu) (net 47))
 (segment (start 179.07 125.73) (end 172.72 119.38) (width 0.25) (layer B.Cu) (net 19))
 (segment (start 172.72 119.38) (end 127 119.38) (width 0.25) (layer B.Cu) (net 19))
 (segment (start 127 119.38) (end 125.73 118.11) (width 0.25) (layer B.Cu) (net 19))
 (segment (start 125.73 87.63) (end 128.27 85.09) (width 0.25) (layer B.Cu) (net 19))
 (segment (start 125.73 118.11) (end 125.73 87.63) (width 0.25) (layer B.Cu) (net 19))
 (segment (start 123.62 85.09) (end 105.99 67.46) (width 0.25) (layer F.Cu) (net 19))
 (segment (start 128.27 85.09) (end 123.62 85.09) (width 0.25) (layer F.Cu) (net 19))
 (segment (start 105.99 60.96) (end 105.99 67.46) (width 0.25) (layer F.Cu) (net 19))
 (segment (start 151.13 95.25) (end 153.67 97.79) (width 0.25) (layer F.Cu) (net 3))
 (segment (start 151.13 87.63) (end 151.13 95.25) (width 0.25) (layer F.Cu) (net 3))
 (segment (start 194.31 57.15) (end 153.67 97.79) (width 0.25) (layer B.Cu) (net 3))
 (segment (start 194.31 57.15) (end 194.31 55.88) (width 0.25) (layer B.Cu) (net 3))
 (segment (start 148.59 95.25) (end 151.13 97.79) (width 0.25) (layer F.Cu) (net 4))
 (segment (start 148.59 87.63) (end 148.59 95.25) (width 0.25) (layer F.Cu) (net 4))
 (segment (start 151.13 97.79) (end 191.77 57.15) (width 0.25) (layer B.Cu) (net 4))
 (segment (start 191.77 57.15) (end 191.77 55.88) (width 0.25) (layer B.Cu) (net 4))
 (segment (start 181.61 100.33) (end 184.15 97.79) (width 0.25) (layer F.Cu) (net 5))
 (segment (start 148.59 100.33) (end 181.61 100.33) (width 0.25) (layer F.Cu) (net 5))
 (segment (start 143.51 95.25) (end 148.59 100.33) (width 0.25) (layer F.Cu) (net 5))
 (segment (start 143.51 87.63) (end 143.51 95.25) (width 0.25) (layer F.Cu) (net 5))
 (segment (start 184.15 97.79) (end 184.15 58.42) (width 0.25) (layer F.Cu) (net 5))
 (segment (start 184.15 58.42) (end 186.69 55.88) (width 0.25) (layer F.Cu) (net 5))
 (segment (start 132.08 91.44) (end 128.27 95.25) (width 0.25) (layer B.Cu) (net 7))
 (segment (start 132.08 82.55) (end 132.08 91.44) (width 0.25) (layer B.Cu) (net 7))
 (segment (start 134.62 80.01) (end 132.08 82.55) (width 0.25) (layer B.Cu) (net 7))
 (segment (start 146.05 80.01) (end 134.62 80.01) (width 0.25) (layer B.Cu) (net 7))
 (segment (start 148.59 77.47) (end 146.05 80.01) (width 0.25) (layer B.Cu) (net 7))
 (segment (start 161.29 74.93) (end 151.13 74.93) (width 0.25) (layer B.Cu) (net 7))
 (segment (start 151.13 74.93) (end 148.59 77.47) (width 0.25) (layer B.Cu) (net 7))
 (segment (start 146.05 82.55) (end 151.13 77.47) (width 0.25) (layer B.Cu) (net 6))
 (segment (start 128.27 97.79) (end 134.62 91.44) (width 0.25) (layer B.Cu) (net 6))
 (segment (start 134.62 85.09) (end 137.16 82.55) (width 0.25) (layer B.Cu) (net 6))
 (segment (start 134.62 91.44) (end 134.62 85.09) (width 0.25) (layer B.Cu) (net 6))
 (segment (start 146.05 82.55) (end 137.16 82.55) (width 0.25) (layer B.Cu) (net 6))
 (segment (start 151.13 77.47) (end 161.29 77.47) (width 0.25) (layer B.Cu) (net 6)))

